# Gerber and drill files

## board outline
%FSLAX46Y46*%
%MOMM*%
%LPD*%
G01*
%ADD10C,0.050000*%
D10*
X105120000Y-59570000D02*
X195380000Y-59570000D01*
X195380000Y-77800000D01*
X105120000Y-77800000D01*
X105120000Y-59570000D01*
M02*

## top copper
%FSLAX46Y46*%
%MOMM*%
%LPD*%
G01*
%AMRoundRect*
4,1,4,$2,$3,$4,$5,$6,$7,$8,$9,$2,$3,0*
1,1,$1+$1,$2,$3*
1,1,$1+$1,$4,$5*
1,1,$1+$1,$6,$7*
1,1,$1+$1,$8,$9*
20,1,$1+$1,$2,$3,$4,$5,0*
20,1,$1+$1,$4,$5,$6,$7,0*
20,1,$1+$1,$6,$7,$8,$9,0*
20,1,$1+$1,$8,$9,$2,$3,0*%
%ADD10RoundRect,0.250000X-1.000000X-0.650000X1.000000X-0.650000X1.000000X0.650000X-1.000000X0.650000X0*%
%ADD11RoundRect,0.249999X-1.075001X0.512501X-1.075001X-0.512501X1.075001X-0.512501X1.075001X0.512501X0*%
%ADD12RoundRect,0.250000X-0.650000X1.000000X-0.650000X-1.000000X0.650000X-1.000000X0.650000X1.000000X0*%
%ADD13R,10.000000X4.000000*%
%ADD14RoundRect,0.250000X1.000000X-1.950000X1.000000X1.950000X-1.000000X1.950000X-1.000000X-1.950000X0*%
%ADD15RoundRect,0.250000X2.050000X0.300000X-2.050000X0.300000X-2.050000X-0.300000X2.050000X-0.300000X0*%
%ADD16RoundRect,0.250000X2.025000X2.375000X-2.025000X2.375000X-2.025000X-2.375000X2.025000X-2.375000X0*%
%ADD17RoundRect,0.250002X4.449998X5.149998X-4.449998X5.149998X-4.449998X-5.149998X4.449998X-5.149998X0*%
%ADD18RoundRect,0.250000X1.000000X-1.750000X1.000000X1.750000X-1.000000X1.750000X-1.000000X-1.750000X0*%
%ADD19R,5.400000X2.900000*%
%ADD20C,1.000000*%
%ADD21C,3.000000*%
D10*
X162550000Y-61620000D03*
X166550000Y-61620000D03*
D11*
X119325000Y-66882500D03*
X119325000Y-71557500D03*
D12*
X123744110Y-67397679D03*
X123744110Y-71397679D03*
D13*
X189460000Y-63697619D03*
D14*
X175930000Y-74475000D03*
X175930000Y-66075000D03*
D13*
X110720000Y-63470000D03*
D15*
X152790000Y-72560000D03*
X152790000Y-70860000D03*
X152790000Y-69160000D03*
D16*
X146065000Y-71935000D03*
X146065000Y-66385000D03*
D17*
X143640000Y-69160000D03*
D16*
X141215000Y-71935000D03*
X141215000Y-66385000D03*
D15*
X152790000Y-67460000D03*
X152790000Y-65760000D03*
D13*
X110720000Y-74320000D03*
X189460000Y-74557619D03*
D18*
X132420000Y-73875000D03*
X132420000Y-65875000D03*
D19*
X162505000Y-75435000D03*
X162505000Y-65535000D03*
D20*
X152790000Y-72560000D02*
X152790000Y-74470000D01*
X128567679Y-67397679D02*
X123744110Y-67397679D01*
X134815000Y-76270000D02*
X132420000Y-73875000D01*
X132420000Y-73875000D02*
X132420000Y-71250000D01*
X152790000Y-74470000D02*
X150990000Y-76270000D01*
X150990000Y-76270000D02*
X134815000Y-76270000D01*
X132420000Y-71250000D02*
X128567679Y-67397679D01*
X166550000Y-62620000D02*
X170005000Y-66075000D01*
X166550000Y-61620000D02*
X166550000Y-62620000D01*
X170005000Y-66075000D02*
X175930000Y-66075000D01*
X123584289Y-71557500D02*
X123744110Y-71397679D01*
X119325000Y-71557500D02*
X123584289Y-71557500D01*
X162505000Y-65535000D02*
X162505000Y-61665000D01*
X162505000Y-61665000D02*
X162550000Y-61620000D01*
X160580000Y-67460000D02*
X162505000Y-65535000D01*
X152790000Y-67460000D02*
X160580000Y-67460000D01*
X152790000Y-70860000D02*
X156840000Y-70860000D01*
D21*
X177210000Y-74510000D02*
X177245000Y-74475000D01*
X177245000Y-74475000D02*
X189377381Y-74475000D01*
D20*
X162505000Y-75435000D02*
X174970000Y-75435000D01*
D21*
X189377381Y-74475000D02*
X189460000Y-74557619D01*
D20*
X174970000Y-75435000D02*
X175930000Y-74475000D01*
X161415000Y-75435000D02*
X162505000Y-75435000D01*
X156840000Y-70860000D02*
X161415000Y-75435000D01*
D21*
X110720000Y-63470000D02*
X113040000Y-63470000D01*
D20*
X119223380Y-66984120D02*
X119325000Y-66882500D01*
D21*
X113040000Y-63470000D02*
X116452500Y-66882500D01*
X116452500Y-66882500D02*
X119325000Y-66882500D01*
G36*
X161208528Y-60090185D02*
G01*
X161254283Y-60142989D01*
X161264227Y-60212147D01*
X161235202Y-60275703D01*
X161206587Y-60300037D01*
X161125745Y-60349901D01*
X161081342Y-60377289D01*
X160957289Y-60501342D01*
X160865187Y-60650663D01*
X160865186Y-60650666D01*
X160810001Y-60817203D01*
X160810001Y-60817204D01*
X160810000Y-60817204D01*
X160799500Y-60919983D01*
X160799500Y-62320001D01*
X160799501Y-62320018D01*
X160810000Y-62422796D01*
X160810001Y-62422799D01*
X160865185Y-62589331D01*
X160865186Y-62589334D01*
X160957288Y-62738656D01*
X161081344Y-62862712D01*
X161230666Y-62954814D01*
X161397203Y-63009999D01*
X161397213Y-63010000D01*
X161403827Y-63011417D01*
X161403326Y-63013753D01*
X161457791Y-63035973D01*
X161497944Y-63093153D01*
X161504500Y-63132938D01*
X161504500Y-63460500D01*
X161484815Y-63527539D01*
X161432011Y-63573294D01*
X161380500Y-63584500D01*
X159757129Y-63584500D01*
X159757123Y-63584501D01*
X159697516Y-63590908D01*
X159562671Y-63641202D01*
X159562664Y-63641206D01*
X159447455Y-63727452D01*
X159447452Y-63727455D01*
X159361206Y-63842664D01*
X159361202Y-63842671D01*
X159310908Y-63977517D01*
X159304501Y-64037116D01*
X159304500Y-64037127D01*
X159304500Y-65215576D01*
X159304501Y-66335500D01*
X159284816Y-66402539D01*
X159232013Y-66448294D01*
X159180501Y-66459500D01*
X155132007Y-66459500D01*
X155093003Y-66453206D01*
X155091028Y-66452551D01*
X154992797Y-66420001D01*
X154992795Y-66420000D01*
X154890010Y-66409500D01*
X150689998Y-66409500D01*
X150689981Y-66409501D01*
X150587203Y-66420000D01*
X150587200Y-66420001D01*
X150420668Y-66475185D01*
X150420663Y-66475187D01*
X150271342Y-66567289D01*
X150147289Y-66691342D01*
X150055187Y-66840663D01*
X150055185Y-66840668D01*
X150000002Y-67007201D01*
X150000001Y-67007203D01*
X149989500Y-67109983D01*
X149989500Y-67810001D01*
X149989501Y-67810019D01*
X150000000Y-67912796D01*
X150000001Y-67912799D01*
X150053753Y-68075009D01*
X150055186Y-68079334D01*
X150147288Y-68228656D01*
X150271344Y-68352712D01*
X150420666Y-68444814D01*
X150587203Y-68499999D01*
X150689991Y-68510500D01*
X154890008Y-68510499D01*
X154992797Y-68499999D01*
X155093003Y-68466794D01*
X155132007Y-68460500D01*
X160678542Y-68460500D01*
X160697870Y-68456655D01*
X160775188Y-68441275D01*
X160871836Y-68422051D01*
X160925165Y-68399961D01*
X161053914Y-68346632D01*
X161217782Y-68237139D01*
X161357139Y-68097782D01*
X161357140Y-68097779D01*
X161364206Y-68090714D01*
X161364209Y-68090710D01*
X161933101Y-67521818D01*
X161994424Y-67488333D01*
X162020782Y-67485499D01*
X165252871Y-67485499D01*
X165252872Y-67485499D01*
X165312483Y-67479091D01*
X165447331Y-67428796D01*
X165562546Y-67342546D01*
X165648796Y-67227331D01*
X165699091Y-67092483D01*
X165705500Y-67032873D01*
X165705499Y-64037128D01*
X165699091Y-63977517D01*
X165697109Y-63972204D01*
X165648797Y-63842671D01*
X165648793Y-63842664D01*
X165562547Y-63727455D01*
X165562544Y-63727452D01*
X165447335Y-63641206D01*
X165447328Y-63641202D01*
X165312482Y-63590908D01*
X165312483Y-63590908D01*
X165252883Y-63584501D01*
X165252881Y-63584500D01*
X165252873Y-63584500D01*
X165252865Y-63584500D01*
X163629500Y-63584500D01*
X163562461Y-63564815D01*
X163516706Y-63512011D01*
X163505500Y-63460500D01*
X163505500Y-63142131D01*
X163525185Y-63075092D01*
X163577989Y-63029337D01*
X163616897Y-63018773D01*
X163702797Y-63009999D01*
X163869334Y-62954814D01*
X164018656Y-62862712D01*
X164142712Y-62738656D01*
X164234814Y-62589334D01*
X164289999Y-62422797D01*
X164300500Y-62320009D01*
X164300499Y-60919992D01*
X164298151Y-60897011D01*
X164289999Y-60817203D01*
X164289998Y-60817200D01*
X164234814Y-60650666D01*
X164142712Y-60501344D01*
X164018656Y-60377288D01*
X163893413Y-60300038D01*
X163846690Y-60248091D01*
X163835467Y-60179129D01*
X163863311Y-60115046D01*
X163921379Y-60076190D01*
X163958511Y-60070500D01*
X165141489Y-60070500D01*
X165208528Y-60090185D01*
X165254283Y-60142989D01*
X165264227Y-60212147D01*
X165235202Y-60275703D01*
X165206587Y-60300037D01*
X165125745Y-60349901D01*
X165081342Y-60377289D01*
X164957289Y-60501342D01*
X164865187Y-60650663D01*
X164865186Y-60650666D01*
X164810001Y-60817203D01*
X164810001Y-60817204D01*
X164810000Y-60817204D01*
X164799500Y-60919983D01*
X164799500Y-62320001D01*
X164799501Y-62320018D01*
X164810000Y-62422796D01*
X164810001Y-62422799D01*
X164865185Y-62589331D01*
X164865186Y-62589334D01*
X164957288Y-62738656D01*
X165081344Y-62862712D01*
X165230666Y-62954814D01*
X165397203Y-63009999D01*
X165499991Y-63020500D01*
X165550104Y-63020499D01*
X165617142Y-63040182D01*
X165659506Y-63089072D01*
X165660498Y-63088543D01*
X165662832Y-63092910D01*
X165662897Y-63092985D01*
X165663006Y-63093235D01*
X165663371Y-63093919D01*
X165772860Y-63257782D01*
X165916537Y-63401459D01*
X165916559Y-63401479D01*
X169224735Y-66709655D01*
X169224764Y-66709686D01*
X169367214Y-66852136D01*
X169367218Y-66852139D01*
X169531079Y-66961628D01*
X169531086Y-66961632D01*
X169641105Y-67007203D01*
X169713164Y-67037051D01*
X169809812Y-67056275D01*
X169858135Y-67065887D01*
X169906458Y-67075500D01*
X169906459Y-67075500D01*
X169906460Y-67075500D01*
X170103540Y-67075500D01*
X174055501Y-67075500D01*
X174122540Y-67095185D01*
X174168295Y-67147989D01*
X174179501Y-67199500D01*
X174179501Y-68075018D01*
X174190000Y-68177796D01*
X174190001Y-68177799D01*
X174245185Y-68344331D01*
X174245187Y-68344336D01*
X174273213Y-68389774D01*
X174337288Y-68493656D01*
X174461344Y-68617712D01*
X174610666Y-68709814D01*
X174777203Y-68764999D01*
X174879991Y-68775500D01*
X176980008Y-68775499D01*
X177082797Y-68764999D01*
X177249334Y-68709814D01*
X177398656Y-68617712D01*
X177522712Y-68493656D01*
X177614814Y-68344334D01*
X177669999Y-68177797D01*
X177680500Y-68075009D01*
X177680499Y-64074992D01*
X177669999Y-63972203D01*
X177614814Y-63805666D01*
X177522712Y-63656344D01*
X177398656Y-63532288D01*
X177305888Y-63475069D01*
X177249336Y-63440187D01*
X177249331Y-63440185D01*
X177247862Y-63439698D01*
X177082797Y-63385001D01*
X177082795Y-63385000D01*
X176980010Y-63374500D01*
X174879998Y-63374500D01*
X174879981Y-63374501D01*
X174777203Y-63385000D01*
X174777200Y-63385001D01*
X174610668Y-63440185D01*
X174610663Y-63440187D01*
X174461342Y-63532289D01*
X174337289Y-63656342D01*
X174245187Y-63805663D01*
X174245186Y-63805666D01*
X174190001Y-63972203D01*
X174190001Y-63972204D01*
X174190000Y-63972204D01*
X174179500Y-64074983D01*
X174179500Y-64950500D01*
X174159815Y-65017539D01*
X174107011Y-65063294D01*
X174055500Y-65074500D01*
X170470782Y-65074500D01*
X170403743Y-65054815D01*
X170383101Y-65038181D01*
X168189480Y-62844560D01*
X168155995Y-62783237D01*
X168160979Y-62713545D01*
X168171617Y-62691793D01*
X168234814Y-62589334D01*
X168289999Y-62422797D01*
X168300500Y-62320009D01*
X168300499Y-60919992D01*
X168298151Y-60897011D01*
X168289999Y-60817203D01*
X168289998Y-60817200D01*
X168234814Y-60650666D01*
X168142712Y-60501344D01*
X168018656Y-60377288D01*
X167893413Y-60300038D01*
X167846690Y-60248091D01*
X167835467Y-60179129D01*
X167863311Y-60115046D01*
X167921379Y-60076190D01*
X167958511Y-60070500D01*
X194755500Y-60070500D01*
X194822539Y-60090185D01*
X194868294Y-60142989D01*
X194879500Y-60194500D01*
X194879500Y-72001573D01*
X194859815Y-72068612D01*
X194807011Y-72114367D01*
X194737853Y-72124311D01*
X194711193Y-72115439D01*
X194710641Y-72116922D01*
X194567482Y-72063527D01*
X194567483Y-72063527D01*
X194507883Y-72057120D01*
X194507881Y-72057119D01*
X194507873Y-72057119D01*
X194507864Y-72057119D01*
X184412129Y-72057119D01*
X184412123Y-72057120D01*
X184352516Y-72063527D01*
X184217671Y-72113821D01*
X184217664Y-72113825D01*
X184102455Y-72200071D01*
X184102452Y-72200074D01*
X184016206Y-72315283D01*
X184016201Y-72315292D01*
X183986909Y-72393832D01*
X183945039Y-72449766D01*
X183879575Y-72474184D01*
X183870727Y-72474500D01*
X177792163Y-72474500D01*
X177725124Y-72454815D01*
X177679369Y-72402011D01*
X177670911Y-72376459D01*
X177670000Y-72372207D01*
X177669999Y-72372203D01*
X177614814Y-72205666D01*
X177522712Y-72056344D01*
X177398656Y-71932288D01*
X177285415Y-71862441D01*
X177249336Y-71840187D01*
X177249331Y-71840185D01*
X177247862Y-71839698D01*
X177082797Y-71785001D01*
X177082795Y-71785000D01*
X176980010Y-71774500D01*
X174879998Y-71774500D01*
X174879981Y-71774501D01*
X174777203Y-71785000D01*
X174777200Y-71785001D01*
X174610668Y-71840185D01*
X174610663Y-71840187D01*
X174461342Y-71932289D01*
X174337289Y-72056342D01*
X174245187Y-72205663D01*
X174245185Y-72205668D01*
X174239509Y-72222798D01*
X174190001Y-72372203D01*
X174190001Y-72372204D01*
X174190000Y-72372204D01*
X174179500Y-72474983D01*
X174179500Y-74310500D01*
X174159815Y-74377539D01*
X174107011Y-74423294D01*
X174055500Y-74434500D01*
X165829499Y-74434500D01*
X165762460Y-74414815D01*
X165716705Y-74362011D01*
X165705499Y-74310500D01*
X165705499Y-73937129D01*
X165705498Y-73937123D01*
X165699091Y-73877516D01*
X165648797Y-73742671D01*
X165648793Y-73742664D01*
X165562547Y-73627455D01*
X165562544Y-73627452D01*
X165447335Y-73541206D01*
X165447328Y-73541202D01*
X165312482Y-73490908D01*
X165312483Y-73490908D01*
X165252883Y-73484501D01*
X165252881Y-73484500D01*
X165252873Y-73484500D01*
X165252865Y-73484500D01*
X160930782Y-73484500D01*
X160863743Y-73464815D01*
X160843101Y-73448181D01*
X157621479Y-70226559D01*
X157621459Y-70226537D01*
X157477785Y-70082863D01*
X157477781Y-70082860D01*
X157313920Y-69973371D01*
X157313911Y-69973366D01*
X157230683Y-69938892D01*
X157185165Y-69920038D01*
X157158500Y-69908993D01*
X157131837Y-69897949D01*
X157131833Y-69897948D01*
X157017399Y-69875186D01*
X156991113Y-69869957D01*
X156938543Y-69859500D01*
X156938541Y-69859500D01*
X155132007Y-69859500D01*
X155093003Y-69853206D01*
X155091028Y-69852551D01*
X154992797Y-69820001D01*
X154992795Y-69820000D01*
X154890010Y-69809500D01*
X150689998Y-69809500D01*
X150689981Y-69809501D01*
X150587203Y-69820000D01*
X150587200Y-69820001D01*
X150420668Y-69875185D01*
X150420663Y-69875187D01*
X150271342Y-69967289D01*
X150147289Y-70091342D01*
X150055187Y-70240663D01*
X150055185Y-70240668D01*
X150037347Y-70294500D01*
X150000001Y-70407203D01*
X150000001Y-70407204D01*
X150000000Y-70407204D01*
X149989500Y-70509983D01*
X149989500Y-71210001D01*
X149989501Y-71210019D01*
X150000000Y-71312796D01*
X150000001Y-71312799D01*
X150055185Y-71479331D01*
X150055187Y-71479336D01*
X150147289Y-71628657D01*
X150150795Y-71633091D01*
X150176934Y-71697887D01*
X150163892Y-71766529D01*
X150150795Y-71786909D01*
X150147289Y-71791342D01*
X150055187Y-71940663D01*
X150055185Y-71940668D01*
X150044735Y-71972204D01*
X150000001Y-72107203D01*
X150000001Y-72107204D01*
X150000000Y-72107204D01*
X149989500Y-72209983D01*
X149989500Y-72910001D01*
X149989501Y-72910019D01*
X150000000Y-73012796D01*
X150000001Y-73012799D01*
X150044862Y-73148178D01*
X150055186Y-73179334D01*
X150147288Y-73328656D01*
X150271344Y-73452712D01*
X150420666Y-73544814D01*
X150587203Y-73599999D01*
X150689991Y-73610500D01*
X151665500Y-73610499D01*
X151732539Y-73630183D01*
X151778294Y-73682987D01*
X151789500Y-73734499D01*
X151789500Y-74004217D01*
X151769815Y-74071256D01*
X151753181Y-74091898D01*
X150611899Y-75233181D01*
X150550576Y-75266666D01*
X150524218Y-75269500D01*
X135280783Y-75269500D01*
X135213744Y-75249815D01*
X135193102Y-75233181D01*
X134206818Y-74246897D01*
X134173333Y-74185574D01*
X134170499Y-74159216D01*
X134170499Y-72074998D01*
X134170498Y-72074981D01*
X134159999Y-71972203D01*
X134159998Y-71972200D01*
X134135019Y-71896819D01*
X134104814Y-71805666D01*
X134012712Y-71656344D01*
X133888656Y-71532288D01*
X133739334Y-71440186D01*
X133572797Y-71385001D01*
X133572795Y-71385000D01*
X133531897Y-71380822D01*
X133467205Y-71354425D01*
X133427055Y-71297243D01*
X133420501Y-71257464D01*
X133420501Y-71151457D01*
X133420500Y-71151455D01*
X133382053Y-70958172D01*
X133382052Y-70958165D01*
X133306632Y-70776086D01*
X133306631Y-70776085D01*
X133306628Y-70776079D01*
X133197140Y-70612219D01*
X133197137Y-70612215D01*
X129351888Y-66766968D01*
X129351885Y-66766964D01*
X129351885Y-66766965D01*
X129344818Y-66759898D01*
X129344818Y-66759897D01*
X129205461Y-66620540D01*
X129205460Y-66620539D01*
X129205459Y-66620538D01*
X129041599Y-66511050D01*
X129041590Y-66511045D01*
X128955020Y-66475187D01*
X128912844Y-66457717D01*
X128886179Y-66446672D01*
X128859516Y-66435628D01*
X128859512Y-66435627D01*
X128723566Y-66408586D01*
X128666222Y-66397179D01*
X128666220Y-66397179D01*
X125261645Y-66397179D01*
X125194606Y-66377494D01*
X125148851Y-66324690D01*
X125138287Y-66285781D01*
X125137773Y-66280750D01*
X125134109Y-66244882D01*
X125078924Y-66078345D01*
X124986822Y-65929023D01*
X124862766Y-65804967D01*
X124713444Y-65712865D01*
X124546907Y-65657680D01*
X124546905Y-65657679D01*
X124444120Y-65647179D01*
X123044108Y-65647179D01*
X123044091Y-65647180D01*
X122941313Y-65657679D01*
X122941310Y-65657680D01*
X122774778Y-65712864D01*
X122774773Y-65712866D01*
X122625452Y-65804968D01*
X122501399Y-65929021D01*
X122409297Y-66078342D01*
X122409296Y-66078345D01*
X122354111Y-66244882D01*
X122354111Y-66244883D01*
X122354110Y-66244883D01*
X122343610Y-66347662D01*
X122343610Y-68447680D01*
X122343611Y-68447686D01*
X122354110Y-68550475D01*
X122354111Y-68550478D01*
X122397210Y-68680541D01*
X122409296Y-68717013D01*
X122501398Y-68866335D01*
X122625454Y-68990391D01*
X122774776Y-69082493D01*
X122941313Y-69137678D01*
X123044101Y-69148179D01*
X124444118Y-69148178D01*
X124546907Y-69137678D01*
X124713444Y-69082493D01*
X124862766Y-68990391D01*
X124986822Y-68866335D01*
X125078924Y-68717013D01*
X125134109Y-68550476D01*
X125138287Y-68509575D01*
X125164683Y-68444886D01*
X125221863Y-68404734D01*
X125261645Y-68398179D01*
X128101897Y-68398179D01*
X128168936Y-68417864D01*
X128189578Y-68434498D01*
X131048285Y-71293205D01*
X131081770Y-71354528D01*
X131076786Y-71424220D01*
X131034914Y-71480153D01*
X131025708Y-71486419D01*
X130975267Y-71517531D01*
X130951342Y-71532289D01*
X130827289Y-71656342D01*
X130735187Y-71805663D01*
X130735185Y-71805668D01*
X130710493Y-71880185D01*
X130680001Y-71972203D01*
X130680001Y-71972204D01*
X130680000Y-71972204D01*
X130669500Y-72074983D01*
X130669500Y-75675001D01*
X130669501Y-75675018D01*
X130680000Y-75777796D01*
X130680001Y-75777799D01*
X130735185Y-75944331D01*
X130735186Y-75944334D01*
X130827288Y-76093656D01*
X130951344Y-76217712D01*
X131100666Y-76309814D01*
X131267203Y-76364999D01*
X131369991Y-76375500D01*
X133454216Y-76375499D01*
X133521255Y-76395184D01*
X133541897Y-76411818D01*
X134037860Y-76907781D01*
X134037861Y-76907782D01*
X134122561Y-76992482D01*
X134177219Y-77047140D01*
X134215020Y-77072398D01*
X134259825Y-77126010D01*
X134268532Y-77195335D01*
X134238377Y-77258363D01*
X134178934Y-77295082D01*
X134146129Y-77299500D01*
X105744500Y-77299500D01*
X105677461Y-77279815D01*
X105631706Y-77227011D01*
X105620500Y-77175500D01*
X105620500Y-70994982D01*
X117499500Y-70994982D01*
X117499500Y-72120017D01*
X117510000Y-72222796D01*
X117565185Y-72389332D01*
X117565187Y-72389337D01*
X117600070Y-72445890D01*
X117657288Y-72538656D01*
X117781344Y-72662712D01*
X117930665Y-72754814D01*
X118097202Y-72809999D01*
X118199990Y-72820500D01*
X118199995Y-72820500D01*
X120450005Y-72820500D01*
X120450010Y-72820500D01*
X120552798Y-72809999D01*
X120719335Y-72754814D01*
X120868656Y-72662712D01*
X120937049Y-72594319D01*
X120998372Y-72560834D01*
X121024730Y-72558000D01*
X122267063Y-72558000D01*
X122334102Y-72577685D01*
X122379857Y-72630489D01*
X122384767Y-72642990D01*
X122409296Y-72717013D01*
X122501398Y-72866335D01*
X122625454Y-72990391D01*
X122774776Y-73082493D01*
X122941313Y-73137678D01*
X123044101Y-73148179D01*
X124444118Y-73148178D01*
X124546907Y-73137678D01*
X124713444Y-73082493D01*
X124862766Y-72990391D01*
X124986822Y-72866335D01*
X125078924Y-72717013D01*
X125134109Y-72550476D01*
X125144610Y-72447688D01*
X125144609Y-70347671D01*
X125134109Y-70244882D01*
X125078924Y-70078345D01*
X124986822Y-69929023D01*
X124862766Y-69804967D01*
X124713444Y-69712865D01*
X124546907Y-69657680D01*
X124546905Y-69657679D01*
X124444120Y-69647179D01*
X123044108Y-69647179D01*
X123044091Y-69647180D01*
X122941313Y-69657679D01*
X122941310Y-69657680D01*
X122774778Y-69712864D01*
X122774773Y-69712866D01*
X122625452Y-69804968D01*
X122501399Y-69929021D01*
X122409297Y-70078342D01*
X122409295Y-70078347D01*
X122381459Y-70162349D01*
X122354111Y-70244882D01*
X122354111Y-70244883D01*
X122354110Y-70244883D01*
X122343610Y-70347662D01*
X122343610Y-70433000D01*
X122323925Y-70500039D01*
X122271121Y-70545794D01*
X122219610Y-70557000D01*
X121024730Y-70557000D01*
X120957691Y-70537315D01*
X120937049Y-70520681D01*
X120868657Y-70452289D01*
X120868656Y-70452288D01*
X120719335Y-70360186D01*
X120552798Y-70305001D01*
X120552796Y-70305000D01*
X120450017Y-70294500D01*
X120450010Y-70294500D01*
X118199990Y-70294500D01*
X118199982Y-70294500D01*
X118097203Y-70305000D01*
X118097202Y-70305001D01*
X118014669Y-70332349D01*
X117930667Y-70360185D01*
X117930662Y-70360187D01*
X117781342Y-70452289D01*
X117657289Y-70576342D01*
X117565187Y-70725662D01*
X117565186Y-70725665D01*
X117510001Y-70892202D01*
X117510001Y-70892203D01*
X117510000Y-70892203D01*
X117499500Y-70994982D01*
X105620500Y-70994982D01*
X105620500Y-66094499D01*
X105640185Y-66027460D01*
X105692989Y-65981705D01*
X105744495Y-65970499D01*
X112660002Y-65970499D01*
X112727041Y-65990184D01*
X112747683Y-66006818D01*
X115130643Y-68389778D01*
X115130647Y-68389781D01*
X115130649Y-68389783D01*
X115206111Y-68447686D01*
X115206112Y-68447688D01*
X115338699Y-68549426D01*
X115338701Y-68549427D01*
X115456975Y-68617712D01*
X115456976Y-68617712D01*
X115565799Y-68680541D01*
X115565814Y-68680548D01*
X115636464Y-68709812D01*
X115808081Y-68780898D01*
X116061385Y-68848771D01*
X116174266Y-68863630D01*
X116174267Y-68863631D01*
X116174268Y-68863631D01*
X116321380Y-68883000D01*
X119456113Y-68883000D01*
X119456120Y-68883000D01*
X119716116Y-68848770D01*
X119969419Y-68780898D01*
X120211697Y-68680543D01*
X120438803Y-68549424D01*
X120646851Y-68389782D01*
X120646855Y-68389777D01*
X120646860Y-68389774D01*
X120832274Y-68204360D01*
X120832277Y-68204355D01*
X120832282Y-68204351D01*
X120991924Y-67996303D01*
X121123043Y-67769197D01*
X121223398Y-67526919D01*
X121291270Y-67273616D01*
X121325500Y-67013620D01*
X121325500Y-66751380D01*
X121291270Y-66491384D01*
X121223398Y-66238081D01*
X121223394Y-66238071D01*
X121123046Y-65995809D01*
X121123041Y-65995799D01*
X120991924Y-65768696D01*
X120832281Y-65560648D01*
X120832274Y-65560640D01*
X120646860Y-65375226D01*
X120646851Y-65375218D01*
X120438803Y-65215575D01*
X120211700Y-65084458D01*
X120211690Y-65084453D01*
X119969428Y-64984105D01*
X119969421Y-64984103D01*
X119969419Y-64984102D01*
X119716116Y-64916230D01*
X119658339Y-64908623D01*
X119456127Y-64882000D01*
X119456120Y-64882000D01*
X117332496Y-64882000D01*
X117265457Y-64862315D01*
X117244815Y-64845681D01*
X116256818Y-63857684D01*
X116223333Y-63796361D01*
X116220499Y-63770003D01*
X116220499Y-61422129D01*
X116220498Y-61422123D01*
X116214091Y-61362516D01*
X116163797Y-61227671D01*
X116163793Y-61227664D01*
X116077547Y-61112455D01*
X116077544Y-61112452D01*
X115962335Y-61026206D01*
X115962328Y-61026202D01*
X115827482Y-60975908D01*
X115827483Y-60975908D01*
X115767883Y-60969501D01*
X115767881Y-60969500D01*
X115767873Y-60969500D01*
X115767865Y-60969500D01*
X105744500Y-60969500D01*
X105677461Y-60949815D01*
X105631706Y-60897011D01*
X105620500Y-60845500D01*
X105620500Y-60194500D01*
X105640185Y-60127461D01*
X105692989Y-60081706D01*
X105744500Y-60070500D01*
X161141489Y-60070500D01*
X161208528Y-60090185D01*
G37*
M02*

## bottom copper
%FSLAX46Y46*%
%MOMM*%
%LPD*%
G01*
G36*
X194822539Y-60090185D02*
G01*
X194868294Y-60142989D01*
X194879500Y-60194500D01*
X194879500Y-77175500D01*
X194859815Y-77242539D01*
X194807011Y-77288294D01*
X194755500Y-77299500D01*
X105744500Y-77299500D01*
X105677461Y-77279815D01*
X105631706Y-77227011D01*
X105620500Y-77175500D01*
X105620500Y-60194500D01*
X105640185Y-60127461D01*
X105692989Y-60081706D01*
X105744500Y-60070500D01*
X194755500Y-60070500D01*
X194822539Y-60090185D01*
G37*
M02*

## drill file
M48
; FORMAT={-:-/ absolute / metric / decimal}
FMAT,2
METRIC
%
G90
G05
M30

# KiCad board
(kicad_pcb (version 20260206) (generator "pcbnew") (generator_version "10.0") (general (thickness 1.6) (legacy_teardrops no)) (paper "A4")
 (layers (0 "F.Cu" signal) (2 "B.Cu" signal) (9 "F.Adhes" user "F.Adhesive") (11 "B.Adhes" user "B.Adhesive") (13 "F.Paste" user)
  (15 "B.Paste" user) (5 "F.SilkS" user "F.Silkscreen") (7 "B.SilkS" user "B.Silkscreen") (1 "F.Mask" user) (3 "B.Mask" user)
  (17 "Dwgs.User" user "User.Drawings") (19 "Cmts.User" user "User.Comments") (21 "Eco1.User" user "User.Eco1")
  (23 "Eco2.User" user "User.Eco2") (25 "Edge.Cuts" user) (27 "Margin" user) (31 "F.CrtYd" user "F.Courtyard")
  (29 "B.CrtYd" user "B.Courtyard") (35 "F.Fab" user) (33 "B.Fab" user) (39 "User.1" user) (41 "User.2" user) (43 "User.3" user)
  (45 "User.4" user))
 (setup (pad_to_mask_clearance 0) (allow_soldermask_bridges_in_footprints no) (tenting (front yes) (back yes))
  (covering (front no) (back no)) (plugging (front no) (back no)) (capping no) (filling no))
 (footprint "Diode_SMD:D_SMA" (layer "F.Cu") (at 164.55 61.62)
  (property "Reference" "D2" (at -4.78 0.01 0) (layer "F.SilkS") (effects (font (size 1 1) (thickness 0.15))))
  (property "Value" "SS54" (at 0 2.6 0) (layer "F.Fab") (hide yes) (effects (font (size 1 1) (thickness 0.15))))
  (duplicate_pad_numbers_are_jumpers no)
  (pad "1" smd roundrect (at -2 0) (size 2.5 1.8) (layers "F.Cu" "F.Mask" "F.Paste") (roundrect_rratio 0.1388888889) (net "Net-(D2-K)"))
  (pad "2" smd roundrect (at 2 0) (size 2.5 1.8) (layers "F.Cu" "F.Mask" "F.Paste") (roundrect_rratio 0.1388888889) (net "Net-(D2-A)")))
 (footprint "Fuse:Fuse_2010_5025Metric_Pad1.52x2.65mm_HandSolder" (layer "F.Cu") (at 119.325 69.22 -90)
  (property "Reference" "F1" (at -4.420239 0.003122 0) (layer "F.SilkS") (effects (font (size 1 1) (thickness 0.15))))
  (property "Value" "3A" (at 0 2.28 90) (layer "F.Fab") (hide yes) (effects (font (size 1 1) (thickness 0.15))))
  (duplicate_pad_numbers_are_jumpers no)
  (pad "1" smd roundrect (at -2.3375 0 270) (size 1.525 2.65) (layers "F.Cu" "F.Mask" "F.Paste") (roundrect_rratio 0.163934) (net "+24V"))
  (pad "2" smd roundrect (at 2.3375 0 270) (size 1.525 2.65) (layers "F.Cu" "F.Mask" "F.Paste") (roundrect_rratio 0.163934)
   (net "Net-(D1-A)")))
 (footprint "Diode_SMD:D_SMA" (layer "F.Cu") (at 123.74411 69.397679 -90)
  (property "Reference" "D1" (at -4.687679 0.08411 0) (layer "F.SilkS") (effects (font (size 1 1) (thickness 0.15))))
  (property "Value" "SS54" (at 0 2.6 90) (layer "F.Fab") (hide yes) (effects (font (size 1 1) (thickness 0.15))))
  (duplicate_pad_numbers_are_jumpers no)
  (pad "1" smd roundrect (at -2 0 270) (size 2.5 1.8) (layers "F.Cu" "F.Mask" "F.Paste") (roundrect_rratio 0.1388888889) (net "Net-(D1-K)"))
  (pad "2" smd roundrect (at 2 0 270) (size 2.5 1.8) (layers "F.Cu" "F.Mask" "F.Paste") (roundrect_rratio 0.1388888889) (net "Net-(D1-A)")))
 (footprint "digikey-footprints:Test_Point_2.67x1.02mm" (layer "F.Cu") (at 189.46 63.697619)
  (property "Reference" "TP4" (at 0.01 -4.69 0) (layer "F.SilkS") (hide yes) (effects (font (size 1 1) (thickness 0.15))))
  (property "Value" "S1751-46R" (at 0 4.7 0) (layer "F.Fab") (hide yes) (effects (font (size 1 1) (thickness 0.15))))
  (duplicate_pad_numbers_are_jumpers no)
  (pad "1" smd rect (at 0 0) (size 10 4) (layers "F.Cu" "F.Mask" "F.Paste") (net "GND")))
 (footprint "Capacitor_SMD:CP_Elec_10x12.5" (layer "F.Cu") (at 175.93 70.275 90)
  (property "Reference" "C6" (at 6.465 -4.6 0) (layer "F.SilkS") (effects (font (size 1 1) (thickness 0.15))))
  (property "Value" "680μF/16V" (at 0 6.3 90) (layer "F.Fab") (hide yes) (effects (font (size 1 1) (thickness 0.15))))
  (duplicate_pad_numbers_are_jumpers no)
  (pad "1" smd roundrect (at -4.2 0 90) (size 4.4 2.5) (layers "F.Cu" "F.Mask" "F.Paste") (roundrect_rratio 0.1) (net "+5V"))
  (pad "2" smd roundrect (at 4.2 0 90) (size 4.4 2.5) (layers "F.Cu" "F.Mask" "F.Paste") (roundrect_rratio 0.1) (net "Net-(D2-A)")))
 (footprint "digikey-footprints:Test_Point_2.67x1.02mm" (layer "F.Cu") (at 110.72 63.47 180)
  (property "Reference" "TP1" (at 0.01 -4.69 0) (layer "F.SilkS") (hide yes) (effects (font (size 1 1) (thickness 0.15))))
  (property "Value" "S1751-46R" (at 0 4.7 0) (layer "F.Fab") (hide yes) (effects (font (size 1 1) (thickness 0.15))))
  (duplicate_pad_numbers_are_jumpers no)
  (pad "1" smd rect (at 0 0 180) (size 10 4) (layers "F.Cu" "F.Mask" "F.Paste") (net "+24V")))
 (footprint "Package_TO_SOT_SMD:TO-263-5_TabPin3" (layer "F.Cu") (at 145.14 69.16 180)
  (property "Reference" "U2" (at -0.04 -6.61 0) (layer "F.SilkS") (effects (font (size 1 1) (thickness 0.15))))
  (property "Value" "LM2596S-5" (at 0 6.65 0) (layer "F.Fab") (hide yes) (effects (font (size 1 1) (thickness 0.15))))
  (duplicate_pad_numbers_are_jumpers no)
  (pad "1" smd roundrect (at -7.65 -3.4 180) (size 4.6 1.1) (layers "F.Cu" "F.Mask" "F.Paste") (roundrect_rratio 0.227273)
   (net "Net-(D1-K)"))
  (pad "2" smd roundrect (at -7.65 -1.7 180) (size 4.6 1.1) (layers "F.Cu" "F.Mask" "F.Paste") (roundrect_rratio 0.227273) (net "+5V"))
  (pad "3" smd roundrect (at -7.65 0 180) (size 4.6 1.1) (layers "F.Cu" "F.Mask" "F.Paste") (roundrect_rratio 0.227273) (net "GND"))
  (pad "3" smd roundrect (at -0.925 -2.775 180) (size 4.55 5.25) (layers "F.Cu" "F.Paste") (roundrect_rratio 0.054945) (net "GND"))
  (pad "3" smd roundrect (at -0.925 2.775 180) (size 4.55 5.25) (layers "F.Cu" "F.Paste") (roundrect_rratio 0.054945) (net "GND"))
  (pad "3" smd roundrect (at 1.5 0 180) (size 9.4 10.8) (layers "F.Cu" "F.Mask") (roundrect_rratio 0.026596) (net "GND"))
  (pad "3" smd roundrect (at 3.925 -2.775 180) (size 4.55 5.25) (layers "F.Cu" "F.Paste") (roundrect_rratio 0.054945) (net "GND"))
  (pad "3" smd roundrect (at 3.925 2.775 180) (size 4.55 5.25) (layers "F.Cu" "F.Paste") (roundrect_rratio 0.054945) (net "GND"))
  (pad "4" smd roundrect (at -7.65 1.7 180) (size 4.6 1.1) (layers "F.Cu" "F.Mask" "F.Paste") (roundrect_rratio 0.227273) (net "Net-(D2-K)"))
  (pad "5" smd roundrect (at -7.65 3.4 180) (size 4.6 1.1) (layers "F.Cu" "F.Mask" "F.Paste") (roundrect_rratio 0.227273) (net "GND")))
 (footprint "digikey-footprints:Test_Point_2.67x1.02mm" (layer "F.Cu") (at 110.72 74.32)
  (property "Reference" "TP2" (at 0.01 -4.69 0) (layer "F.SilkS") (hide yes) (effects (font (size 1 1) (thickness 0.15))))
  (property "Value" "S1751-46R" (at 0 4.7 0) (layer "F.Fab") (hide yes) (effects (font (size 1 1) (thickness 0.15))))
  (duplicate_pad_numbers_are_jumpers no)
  (pad "1" smd rect (at 0 0) (size 10 4) (layers "F.Cu" "F.Mask" "F.Paste") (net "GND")))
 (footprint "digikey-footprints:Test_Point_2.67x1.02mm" (layer "F.Cu") (at 189.46 74.557619)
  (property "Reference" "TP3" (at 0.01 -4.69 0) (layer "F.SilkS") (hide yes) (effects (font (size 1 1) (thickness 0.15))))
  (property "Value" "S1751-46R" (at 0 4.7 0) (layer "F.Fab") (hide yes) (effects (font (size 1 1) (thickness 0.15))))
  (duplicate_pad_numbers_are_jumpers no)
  (pad "1" smd rect (at 0 0) (size 10 4) (layers "F.Cu" "F.Mask" "F.Paste") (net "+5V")))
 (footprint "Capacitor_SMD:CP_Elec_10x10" (layer "F.Cu") (at 132.42 69.875 90)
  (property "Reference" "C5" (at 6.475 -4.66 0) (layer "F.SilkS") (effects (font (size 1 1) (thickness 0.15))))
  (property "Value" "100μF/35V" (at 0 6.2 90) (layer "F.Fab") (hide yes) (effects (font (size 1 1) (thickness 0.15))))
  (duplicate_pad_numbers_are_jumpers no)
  (pad "1" smd roundrect (at -4 0 90) (size 4 2.5) (layers "F.Cu" "F.Mask" "F.Paste") (roundrect_rratio 0.1) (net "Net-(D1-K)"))
  (pad "2" smd roundrect (at 4 0 90) (size 4 2.5) (layers "F.Cu" "F.Mask" "F.Paste") (roundrect_rratio 0.1) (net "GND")))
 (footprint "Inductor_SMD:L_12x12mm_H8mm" (layer "F.Cu") (at 162.505 70.485 90)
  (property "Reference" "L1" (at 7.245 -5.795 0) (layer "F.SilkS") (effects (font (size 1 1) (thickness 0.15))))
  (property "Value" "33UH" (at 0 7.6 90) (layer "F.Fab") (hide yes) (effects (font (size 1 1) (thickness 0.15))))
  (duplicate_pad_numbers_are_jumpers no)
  (pad "1" smd rect (at -4.95 0 90) (size 2.9 5.4) (layers "F.Cu" "F.Mask" "F.Paste") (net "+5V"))
  (pad "2" smd rect (at 4.95 0 90) (size 2.9 5.4) (layers "F.Cu" "F.Mask" "F.Paste") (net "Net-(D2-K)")))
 (gr_rect (start 105.12 59.57) (end 195.38 77.8) (stroke (width 0.05) (type default)) (fill no) (layer "Edge.Cuts"))
 (segment (start 152.79 72.56) (end 152.79 74.47) (width 1) (layer "F.Cu") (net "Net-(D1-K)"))
 (segment (start 128.567679 67.397679) (end 123.74411 67.397679) (width 1) (layer "F.Cu") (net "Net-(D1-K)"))
 (segment (start 134.815 76.27) (end 132.42 73.875) (width 1) (layer "F.Cu") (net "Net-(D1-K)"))
 (segment (start 132.42 73.875) (end 132.42 71.25) (width 1) (layer "F.Cu") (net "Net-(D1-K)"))
 (segment (start 152.79 74.47) (end 150.99 76.27) (width 1) (layer "F.Cu") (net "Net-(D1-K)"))
 (segment (start 150.99 76.27) (end 134.815 76.27) (width 1) (layer "F.Cu") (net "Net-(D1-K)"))
 (segment (start 132.42 71.25) (end 128.567679 67.397679) (width 1) (layer "F.Cu") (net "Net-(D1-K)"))
 (segment (start 166.55 62.62) (end 170.005 66.075) (width 1) (layer "F.Cu") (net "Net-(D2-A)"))
 (segment (start 166.55 61.62) (end 166.55 62.62) (width 1) (layer "F.Cu") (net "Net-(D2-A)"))
 (segment (start 170.005 66.075) (end 175.93 66.075) (width 1) (layer "F.Cu") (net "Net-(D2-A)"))
 (segment (start 123.584289 71.5575) (end 123.74411 71.397679) (width 1) (layer "F.Cu") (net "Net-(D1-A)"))
 (segment (start 119.325 71.5575) (end 123.584289 71.5575) (width 1) (layer "F.Cu") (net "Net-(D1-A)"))
 (segment (start 162.505 65.535) (end 162.505 61.665) (width 1) (layer "F.Cu") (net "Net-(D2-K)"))
 (segment (start 162.505 61.665) (end 162.55 61.62) (width 1) (layer "F.Cu") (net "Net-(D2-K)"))
 (segment (start 160.58 67.46) (end 162.505 65.535) (width 1) (layer "F.Cu") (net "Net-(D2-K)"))
 (segment (start 152.79 67.46) (end 160.58 67.46) (width 1) (layer "F.Cu") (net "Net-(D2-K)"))
 (segment (start 152.79 70.86) (end 156.84 70.86) (width 1) (layer "F.Cu") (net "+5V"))
 (segment (start 177.21 74.51) (end 177.245 74.475) (width 3) (layer "F.Cu") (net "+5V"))
 (segment (start 177.245 74.475) (end 189.377381 74.475) (width 3) (layer "F.Cu") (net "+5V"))
 (segment (start 162.505 75.435) (end 174.97 75.435) (width 1) (layer "F.Cu") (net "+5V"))
 (segment (start 189.377381 74.475) (end 189.46 74.557619) (width 3) (layer "F.Cu") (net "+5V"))
 (segment (start 174.97 75.435) (end 175.93 74.475) (width 1) (layer "F.Cu") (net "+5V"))
 (segment (start 161.415 75.435) (end 162.505 75.435) (width 1) (layer "F.Cu") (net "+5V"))
 (segment (start 156.84 70.86) (end 161.415 75.435) (width 1) (layer "F.Cu") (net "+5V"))
 (segment (start 110.72 63.47) (end 113.04 63.47) (width 3) (layer "F.Cu") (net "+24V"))
 (segment (start 119.22338 66.98412) (end 119.325 66.8825) (width 1) (layer "F.Cu") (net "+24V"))
 (segment (start 113.04 63.47) (end 116.4525 66.8825) (width 3) (layer "F.Cu") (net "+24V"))
 (segment (start 116.4525 66.8825) (end 119.325 66.8825) (width 3) (layer "F.Cu") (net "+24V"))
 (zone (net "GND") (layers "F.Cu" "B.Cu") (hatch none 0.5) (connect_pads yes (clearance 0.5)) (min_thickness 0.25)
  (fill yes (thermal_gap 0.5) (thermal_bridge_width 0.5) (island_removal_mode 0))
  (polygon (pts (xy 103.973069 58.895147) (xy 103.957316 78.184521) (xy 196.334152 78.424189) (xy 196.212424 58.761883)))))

